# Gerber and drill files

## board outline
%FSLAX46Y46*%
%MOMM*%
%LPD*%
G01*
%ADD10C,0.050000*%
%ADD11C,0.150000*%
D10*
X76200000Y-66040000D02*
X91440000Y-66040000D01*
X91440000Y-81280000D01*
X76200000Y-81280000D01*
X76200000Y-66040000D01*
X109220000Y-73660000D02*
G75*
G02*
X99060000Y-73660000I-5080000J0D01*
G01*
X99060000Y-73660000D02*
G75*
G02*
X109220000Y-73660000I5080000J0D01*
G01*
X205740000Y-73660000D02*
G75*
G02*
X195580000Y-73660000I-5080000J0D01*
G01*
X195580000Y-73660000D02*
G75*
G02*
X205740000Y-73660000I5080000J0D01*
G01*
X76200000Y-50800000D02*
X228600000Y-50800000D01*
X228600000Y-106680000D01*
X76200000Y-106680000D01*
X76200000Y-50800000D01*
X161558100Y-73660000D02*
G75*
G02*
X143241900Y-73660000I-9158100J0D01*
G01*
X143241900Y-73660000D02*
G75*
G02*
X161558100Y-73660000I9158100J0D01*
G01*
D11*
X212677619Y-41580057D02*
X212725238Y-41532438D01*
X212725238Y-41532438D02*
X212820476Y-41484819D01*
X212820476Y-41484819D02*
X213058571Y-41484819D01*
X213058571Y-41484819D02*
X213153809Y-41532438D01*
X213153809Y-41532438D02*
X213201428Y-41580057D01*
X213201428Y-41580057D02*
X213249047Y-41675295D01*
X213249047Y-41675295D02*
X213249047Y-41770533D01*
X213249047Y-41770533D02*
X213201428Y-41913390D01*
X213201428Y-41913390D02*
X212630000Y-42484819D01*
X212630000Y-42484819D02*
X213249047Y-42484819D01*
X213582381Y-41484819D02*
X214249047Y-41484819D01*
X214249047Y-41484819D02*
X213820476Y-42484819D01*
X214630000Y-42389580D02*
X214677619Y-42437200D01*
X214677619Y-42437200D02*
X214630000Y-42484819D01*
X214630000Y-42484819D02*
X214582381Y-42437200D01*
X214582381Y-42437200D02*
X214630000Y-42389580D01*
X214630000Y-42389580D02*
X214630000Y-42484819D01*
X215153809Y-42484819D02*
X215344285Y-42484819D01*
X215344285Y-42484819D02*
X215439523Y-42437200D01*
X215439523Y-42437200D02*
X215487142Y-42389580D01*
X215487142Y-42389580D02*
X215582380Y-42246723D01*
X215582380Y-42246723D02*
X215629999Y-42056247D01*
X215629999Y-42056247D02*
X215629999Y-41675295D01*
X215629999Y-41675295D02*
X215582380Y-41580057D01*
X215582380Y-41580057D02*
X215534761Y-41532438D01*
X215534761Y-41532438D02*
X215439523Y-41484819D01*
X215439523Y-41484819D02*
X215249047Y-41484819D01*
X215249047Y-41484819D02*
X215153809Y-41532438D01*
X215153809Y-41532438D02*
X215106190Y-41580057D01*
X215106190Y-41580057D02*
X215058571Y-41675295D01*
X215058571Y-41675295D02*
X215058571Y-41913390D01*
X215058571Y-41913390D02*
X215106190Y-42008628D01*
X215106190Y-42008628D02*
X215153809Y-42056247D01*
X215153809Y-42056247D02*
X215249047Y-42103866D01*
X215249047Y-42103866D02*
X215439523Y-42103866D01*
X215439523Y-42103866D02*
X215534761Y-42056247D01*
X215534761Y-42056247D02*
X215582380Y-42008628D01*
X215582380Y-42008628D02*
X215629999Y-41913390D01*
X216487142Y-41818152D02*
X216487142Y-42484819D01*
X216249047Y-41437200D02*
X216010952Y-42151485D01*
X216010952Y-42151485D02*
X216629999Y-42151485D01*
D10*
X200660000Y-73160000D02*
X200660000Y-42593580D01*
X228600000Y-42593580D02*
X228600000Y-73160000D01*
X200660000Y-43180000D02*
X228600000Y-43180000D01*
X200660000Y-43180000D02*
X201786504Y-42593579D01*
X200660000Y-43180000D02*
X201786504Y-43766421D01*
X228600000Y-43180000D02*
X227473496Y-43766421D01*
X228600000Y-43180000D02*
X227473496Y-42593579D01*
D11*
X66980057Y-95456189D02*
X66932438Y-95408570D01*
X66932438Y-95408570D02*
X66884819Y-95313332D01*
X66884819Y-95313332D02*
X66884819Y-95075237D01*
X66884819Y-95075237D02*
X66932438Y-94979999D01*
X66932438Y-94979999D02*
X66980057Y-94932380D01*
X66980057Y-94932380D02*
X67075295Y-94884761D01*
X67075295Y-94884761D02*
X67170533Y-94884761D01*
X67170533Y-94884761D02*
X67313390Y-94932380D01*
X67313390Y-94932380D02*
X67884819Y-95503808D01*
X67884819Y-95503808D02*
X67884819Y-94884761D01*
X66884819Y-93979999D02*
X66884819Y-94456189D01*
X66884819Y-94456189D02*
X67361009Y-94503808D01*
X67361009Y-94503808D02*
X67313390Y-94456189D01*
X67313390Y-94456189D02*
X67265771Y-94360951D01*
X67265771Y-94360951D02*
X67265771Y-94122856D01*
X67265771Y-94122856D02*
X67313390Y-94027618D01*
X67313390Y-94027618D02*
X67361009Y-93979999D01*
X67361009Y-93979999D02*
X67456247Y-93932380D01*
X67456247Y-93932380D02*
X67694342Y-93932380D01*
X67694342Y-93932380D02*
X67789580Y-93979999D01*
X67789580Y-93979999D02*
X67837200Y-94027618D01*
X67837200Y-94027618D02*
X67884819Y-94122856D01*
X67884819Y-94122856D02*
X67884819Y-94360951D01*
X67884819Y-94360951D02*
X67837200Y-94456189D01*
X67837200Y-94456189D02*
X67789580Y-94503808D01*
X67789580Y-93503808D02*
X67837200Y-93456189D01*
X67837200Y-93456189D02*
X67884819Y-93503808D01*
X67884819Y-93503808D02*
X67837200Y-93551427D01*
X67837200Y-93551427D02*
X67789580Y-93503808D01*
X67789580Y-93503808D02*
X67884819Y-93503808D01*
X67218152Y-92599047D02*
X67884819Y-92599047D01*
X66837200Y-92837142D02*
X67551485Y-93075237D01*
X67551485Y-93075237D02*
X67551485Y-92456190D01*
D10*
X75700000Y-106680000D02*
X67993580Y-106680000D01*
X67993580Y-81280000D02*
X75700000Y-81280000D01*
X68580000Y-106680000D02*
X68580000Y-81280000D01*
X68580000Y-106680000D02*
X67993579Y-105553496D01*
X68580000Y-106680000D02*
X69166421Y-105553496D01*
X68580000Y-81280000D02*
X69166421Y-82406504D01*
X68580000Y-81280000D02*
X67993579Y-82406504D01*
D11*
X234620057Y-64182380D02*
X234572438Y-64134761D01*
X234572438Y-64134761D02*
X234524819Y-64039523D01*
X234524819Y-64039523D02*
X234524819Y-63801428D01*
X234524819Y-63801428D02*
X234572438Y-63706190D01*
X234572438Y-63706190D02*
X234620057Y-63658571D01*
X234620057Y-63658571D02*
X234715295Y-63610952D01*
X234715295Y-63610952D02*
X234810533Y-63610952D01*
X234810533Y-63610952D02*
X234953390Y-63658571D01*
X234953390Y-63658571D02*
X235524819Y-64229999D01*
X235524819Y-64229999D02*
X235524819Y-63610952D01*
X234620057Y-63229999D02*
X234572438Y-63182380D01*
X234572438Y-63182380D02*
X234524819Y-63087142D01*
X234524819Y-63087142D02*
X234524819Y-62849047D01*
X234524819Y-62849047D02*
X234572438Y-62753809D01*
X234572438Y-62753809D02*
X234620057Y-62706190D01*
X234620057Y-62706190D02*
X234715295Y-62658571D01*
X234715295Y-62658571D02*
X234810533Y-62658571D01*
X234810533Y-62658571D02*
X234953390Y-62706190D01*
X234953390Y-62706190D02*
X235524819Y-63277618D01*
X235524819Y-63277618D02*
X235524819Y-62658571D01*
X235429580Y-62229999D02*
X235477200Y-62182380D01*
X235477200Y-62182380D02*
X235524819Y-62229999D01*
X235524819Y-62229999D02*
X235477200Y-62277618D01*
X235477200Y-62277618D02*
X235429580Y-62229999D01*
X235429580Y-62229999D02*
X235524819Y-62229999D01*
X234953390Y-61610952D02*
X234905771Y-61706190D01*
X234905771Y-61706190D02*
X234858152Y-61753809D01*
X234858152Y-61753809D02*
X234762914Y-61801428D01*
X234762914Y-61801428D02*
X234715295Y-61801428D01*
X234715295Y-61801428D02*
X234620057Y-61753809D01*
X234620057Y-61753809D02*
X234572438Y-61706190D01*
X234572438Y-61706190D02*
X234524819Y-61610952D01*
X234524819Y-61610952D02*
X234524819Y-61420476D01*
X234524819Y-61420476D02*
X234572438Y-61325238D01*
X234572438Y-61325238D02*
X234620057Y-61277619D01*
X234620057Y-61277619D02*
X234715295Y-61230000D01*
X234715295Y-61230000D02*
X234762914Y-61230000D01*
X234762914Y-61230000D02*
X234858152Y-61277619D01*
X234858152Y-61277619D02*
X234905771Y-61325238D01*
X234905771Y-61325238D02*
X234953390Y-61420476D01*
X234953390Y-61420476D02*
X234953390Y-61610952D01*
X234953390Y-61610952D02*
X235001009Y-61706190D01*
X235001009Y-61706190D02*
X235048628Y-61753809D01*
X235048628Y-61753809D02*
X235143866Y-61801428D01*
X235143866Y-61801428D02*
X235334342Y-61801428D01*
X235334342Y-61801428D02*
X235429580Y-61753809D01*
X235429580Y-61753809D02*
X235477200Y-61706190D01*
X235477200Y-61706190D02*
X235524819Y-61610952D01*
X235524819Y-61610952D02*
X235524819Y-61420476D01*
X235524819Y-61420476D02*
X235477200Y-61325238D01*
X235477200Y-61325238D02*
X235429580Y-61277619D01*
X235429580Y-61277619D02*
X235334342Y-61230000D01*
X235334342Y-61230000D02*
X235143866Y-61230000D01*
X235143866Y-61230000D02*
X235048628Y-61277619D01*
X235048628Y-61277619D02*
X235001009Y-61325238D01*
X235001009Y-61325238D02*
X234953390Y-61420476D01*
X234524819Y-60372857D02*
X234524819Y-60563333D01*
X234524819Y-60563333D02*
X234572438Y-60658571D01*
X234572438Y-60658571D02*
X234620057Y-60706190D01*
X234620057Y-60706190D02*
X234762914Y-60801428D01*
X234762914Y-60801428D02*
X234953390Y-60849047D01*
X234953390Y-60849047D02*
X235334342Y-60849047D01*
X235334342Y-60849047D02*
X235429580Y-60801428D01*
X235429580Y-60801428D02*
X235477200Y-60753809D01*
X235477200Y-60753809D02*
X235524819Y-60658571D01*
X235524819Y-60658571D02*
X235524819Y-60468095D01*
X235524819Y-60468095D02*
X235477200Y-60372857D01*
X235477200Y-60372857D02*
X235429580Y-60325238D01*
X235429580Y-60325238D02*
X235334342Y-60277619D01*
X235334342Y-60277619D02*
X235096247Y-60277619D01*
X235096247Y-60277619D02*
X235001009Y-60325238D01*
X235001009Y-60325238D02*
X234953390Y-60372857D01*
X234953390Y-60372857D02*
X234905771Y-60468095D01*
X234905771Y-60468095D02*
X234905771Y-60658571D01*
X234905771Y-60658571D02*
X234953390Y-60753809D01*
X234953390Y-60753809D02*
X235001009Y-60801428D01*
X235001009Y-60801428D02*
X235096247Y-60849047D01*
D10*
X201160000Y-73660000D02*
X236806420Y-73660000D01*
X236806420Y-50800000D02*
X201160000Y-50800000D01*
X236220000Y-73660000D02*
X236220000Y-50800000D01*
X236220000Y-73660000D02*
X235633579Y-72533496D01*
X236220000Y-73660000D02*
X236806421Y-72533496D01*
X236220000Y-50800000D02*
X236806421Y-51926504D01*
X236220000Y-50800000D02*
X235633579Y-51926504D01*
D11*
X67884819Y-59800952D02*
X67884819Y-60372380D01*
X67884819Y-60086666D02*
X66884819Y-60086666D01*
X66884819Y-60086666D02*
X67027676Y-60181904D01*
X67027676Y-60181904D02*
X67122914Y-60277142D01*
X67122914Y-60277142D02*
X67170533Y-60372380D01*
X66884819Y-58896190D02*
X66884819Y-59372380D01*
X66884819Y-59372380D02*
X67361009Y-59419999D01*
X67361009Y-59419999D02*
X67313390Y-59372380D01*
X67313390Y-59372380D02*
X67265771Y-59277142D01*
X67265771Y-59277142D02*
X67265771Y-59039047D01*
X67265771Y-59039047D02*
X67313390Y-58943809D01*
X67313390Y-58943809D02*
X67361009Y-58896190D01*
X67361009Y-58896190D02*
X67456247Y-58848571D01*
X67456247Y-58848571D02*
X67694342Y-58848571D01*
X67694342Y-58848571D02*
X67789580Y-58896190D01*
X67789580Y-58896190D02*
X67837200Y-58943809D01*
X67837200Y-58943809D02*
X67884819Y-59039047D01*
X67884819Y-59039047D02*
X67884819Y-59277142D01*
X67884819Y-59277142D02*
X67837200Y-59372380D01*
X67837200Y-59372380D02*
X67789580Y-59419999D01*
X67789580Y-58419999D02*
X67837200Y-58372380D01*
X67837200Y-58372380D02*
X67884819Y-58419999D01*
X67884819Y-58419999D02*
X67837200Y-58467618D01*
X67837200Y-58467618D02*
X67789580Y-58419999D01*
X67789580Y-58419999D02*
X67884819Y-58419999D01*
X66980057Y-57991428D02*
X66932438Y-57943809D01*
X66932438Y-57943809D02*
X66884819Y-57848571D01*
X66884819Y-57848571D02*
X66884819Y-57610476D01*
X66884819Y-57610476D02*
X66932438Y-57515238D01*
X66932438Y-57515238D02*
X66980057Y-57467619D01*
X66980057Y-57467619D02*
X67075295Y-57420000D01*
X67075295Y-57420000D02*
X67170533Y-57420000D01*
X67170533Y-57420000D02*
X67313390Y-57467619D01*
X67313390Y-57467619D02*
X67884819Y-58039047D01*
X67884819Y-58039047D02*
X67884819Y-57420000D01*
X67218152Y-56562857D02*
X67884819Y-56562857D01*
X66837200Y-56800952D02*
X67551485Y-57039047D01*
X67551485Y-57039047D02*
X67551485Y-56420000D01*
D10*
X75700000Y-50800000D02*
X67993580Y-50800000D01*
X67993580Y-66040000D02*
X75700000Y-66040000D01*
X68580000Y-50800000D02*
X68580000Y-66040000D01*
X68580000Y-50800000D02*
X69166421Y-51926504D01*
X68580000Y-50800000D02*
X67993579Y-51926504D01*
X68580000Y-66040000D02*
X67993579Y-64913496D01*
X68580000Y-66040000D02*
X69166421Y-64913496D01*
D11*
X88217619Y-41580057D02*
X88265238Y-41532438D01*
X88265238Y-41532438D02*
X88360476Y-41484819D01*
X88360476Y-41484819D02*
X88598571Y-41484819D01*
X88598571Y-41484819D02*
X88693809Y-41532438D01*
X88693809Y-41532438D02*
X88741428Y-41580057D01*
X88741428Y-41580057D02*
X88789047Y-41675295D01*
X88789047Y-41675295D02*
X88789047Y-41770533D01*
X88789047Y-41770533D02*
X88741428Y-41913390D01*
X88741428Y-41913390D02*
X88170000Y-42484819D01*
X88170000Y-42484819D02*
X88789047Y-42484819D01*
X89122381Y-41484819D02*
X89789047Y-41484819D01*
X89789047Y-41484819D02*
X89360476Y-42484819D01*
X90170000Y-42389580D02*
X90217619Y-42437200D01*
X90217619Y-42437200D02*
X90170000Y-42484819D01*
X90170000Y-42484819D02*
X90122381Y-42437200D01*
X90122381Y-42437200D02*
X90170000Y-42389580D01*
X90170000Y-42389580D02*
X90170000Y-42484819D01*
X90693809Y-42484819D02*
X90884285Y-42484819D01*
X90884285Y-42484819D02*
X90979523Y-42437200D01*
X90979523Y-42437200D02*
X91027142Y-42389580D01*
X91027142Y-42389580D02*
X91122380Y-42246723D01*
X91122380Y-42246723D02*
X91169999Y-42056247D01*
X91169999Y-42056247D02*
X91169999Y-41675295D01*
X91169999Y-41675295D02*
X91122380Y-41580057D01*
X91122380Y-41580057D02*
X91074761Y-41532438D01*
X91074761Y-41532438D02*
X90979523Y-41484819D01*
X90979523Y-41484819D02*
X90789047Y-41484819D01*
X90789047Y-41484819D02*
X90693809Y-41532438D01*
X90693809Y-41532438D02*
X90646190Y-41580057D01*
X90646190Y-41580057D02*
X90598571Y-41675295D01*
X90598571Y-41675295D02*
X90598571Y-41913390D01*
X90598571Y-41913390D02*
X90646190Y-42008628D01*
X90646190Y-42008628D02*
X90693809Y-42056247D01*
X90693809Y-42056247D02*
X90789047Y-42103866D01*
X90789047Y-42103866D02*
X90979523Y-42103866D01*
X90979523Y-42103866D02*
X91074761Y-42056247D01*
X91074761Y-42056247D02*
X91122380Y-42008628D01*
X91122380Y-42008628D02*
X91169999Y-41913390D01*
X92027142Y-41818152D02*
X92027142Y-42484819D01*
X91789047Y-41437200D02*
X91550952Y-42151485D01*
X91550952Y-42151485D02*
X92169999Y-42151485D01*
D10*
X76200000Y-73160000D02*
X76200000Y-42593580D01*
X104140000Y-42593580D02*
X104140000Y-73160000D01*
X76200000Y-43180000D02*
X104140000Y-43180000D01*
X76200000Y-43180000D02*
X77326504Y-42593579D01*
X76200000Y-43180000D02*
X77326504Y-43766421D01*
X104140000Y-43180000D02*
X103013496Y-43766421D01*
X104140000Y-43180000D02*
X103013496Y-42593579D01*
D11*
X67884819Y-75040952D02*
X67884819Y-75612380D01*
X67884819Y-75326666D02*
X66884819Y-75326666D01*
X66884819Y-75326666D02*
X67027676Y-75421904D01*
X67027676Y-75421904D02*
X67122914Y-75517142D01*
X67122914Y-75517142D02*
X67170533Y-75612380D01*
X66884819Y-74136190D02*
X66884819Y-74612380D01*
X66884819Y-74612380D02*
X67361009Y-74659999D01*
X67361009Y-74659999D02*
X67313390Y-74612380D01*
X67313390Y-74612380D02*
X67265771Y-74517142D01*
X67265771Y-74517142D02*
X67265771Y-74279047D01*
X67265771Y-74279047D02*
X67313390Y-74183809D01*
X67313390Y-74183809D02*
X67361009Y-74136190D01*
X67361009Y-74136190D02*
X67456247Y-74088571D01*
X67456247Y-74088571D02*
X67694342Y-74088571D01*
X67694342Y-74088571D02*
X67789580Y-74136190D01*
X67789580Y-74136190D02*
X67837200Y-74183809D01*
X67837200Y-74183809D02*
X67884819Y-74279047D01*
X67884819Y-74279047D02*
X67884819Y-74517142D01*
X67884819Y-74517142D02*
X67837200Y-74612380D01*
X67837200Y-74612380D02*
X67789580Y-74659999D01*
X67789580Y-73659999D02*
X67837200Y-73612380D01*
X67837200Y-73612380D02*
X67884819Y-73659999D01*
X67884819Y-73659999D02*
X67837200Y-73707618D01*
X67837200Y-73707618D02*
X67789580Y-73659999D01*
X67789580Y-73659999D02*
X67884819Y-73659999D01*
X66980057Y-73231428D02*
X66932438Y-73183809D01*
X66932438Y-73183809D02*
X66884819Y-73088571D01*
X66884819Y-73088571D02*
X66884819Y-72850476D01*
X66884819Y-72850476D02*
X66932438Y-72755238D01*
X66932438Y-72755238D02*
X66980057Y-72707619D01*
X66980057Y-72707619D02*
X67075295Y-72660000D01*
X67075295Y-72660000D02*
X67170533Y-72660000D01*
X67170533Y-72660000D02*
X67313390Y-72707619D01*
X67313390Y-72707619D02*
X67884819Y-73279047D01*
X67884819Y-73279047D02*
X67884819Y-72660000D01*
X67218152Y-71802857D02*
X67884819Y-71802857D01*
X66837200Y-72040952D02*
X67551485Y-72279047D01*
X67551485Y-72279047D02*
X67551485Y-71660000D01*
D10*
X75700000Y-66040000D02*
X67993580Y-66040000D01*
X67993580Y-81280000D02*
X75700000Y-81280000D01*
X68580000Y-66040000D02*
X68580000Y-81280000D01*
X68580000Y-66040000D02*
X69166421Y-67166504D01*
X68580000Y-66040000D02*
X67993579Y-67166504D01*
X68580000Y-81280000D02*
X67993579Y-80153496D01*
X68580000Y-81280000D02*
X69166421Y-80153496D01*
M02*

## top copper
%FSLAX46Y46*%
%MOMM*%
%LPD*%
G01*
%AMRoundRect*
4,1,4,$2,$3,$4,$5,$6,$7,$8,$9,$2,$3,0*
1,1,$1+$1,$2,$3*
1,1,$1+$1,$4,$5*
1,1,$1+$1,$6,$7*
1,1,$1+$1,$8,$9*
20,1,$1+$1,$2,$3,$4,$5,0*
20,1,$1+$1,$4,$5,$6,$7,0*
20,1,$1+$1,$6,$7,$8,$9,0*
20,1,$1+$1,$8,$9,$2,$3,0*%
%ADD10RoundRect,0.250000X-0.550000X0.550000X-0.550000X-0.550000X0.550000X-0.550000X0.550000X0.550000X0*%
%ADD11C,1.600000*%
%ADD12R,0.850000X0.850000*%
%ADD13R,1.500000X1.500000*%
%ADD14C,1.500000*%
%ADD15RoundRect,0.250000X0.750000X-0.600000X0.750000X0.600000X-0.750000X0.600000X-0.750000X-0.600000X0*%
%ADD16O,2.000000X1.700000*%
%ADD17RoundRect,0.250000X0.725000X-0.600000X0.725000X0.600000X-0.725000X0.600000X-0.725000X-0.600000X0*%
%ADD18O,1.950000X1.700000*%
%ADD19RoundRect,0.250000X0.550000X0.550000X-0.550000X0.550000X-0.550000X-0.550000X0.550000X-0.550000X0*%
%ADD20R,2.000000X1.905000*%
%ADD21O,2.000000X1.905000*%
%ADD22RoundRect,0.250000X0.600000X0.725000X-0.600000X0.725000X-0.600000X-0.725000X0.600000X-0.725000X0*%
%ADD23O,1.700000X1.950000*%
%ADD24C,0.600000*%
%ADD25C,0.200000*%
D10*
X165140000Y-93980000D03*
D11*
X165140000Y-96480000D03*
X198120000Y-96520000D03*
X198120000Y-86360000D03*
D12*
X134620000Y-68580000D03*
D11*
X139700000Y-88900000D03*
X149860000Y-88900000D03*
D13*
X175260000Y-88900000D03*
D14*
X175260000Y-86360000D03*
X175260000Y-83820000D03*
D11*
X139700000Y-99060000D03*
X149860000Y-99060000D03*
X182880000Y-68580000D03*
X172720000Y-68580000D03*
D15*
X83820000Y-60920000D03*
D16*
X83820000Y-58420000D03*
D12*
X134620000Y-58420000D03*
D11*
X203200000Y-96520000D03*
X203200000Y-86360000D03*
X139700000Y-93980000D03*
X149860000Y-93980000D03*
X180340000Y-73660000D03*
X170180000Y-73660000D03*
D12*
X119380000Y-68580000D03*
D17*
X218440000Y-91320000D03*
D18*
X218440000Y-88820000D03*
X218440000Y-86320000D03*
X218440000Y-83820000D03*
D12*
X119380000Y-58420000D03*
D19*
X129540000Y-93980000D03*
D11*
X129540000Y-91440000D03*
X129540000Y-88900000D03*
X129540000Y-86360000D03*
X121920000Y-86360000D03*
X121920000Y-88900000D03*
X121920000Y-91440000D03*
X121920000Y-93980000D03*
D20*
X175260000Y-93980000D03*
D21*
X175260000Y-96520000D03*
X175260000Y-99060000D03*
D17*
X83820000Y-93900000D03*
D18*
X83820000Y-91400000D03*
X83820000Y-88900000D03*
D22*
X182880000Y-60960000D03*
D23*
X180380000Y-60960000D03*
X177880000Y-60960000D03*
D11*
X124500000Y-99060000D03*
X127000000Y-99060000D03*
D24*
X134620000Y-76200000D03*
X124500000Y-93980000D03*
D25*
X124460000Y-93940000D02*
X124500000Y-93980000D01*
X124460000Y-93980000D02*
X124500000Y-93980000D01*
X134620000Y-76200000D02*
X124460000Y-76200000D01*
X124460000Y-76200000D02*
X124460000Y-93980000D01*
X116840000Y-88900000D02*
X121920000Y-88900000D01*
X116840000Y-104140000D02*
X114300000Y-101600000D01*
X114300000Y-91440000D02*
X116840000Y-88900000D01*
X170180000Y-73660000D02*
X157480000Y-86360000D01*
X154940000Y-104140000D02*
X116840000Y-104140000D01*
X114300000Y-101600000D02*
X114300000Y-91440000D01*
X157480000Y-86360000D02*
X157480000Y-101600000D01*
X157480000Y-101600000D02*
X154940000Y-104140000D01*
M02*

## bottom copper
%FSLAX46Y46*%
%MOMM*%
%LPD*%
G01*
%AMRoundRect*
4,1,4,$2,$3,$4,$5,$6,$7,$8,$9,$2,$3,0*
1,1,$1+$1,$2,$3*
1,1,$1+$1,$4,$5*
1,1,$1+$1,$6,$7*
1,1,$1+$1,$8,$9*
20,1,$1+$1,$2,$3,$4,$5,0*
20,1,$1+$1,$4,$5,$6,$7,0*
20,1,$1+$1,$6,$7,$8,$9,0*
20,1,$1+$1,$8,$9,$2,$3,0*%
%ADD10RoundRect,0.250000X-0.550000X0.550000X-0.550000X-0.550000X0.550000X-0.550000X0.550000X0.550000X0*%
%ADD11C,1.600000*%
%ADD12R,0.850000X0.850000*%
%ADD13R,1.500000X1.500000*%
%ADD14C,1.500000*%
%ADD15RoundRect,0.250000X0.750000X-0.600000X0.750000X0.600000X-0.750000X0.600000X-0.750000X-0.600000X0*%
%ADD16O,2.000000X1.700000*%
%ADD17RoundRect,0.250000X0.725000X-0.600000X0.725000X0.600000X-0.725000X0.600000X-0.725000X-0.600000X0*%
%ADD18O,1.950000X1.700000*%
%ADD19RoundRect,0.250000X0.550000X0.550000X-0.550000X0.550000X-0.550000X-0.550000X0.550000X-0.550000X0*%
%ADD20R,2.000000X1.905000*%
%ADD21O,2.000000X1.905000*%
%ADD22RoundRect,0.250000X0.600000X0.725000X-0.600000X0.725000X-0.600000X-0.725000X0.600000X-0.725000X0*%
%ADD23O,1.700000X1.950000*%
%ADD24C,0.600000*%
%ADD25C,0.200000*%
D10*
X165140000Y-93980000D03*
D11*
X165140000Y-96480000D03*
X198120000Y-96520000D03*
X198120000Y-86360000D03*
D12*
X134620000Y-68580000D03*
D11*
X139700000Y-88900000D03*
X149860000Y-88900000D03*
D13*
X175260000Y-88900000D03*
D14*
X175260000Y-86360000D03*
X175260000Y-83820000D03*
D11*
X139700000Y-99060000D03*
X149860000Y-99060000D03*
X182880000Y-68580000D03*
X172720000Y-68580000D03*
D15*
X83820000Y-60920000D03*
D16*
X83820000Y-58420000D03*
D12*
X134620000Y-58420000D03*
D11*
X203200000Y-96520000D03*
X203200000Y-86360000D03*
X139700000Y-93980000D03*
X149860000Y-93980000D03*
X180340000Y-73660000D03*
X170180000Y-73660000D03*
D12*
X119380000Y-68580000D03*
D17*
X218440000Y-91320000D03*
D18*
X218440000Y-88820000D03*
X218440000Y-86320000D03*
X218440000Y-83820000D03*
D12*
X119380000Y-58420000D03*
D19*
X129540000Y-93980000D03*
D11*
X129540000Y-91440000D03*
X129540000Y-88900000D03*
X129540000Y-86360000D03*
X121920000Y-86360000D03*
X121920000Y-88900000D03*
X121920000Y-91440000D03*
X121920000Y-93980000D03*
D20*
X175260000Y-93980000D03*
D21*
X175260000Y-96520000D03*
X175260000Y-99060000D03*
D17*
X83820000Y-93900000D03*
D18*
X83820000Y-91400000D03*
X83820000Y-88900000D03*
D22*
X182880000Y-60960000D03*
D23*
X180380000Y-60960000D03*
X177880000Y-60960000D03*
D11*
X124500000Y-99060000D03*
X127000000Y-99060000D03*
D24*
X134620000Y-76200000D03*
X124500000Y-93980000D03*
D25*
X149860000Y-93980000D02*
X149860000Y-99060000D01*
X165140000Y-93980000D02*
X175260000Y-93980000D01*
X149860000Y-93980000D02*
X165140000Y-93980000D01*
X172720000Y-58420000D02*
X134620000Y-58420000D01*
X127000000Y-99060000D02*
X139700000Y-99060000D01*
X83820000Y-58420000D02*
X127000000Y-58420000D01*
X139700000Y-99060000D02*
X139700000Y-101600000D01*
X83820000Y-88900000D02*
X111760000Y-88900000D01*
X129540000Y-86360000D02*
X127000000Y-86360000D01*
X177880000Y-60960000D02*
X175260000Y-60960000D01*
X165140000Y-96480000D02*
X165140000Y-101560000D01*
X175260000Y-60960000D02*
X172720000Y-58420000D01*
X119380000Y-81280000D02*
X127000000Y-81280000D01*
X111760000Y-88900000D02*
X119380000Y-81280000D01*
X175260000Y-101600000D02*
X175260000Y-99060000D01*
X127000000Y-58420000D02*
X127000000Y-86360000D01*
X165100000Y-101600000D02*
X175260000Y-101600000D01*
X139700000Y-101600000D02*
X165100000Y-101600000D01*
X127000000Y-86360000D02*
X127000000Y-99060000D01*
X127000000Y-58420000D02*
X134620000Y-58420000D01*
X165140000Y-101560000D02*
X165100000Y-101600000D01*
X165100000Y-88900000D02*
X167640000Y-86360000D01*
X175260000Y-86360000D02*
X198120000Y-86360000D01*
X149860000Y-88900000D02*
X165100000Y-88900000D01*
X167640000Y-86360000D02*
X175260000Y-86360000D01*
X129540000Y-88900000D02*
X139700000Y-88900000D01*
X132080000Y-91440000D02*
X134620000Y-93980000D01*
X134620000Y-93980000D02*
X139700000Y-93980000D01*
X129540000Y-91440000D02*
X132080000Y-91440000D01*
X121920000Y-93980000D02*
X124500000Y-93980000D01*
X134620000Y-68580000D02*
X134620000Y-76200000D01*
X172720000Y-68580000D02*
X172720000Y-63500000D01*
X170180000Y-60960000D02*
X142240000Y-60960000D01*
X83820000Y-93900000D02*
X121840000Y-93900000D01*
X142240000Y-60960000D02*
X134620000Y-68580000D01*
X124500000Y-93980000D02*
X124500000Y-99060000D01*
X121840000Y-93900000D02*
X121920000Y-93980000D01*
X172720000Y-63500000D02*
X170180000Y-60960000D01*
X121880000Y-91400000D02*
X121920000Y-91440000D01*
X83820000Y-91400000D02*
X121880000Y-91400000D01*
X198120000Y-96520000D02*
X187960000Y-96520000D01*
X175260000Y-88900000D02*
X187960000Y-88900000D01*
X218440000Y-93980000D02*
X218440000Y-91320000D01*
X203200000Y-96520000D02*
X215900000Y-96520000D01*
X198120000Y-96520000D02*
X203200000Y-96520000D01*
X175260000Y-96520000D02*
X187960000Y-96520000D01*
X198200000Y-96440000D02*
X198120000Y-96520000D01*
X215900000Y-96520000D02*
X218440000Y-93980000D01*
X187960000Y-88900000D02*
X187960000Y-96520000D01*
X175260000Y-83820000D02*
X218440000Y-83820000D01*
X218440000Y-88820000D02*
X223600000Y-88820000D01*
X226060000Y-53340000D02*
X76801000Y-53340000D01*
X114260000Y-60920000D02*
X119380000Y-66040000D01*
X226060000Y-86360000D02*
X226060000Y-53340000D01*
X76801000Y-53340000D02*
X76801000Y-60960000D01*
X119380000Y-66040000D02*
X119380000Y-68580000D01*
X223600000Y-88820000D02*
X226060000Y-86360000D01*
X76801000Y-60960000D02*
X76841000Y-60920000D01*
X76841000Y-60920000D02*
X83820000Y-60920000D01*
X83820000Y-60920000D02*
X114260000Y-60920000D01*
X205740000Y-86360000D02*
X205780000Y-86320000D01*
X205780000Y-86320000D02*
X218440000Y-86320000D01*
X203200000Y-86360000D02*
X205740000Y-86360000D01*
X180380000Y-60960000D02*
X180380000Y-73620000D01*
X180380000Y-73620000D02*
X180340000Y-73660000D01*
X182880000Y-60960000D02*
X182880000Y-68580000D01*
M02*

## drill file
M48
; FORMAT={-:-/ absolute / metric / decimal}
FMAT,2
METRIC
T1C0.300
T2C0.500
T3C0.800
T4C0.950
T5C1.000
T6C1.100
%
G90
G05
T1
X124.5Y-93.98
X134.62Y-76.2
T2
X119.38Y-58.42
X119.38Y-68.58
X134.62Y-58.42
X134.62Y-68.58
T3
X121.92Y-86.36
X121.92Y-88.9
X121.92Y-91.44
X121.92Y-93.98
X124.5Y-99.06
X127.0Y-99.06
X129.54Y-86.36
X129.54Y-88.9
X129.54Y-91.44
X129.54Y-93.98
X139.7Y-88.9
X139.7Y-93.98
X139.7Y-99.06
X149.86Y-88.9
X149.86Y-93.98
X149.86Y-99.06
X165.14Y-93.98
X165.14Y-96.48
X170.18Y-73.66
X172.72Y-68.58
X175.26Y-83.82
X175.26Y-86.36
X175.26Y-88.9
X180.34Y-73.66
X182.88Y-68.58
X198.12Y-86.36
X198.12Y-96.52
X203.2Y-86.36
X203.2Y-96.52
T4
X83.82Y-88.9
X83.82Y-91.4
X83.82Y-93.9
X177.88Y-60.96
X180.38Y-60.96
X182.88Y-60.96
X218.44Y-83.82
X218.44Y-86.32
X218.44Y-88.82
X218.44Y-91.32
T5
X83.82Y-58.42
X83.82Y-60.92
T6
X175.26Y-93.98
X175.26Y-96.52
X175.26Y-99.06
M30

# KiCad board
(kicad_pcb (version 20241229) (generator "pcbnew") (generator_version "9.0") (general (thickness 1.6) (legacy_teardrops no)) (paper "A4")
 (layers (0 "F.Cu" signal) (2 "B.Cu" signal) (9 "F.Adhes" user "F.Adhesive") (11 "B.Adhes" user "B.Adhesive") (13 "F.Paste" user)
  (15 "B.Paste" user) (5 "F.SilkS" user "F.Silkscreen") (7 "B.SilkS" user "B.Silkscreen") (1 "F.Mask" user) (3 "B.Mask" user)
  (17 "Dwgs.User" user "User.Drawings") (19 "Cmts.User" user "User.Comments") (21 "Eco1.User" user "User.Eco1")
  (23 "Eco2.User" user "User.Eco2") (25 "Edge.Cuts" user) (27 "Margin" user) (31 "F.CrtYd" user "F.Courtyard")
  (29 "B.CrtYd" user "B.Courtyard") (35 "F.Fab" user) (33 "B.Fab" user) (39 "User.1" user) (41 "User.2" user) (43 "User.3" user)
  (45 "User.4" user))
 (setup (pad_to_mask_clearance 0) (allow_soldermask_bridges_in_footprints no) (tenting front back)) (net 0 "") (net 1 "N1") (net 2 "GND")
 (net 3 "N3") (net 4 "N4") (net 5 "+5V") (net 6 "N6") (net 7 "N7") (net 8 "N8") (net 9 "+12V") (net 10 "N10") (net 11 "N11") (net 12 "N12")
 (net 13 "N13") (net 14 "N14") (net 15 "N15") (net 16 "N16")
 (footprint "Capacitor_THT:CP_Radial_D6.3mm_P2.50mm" (layer "F.Cu") (at 165.14 93.98 -90)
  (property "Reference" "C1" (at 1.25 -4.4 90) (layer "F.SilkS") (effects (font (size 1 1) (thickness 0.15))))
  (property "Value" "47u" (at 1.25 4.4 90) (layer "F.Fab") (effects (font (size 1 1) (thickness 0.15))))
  (pad "1" thru_hole roundrect (at 0 0 270) (size 1.6 1.6) (drill 0.8) (layers "*.Cu" "*.Mask") (remove_unused_layers no)
   (roundrect_rratio 0.15625) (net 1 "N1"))
  (pad "2" thru_hole circle (at 2.5 0 270) (size 1.6 1.6) (drill 0.8) (layers "*.Cu" "*.Mask") (remove_unused_layers no) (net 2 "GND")))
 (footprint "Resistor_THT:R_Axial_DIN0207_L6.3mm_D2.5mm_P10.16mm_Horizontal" (layer "F.Cu") (at 198.12 96.52 90)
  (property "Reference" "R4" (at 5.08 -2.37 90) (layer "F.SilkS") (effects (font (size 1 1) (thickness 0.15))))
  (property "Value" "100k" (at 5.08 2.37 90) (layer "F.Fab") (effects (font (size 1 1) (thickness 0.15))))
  (pad "1" thru_hole circle (at 0 0 90) (size 1.6 1.6) (drill 0.8) (layers "*.Cu" "*.Mask") (remove_unused_layers no) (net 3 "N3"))
  (pad "2" thru_hole circle (at 10.16 0 90) (size 1.6 1.6) (drill 0.8) (layers "*.Cu" "*.Mask") (remove_unused_layers no) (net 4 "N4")))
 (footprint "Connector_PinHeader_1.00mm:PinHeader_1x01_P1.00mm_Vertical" (layer "F.Cu") (at 134.62 68.58)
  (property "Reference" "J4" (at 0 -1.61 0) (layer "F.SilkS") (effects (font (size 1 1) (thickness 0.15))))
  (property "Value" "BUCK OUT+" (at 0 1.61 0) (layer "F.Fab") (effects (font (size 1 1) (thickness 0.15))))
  (pad "1" thru_hole rect (at 0 0) (size 0.85 0.85) (drill 0.5) (layers "*.Cu" "*.Mask") (remove_unused_layers no) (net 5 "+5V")))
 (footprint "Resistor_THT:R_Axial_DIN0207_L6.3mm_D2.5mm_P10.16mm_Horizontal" (layer "F.Cu") (at 139.7 88.9)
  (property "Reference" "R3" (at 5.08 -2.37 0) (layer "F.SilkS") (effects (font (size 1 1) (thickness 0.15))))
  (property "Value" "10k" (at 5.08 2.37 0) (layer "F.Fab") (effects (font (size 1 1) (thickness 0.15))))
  (pad "1" thru_hole circle (at 0 0) (size 1.6 1.6) (drill 0.8) (layers "*.Cu" "*.Mask") (remove_unused_layers no) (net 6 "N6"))
  (pad "2" thru_hole circle (at 10.16 0) (size 1.6 1.6) (drill 0.8) (layers "*.Cu" "*.Mask") (remove_unused_layers no) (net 4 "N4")))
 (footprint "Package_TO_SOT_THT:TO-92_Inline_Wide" (layer "F.Cu") (at 175.26 88.9 90)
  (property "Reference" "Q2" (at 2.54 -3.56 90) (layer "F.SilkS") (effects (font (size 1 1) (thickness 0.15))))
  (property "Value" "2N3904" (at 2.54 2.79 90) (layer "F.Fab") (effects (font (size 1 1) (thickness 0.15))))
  (pad "1" thru_hole rect (at 0 0 90) (size 1.5 1.5) (drill 0.8) (layers "*.Cu" "*.Mask") (remove_unused_layers no) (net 3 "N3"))
  (pad "2" thru_hole circle (at 2.54 0 90) (size 1.5 1.5) (drill 0.8) (layers "*.Cu" "*.Mask") (remove_unused_layers no) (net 4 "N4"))
  (pad "3" thru_hole circle (at 5.08 0 90) (size 1.5 1.5) (drill 0.8) (layers "*.Cu" "*.Mask") (remove_unused_layers no) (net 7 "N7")))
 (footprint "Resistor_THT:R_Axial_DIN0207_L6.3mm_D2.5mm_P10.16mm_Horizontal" (layer "F.Cu") (at 139.7 99.06)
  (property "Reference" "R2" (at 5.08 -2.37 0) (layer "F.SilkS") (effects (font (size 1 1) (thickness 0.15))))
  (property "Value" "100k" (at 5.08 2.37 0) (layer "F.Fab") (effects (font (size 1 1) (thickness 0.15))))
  (pad "1" thru_hole circle (at 0 0) (size 1.6 1.6) (drill 0.8) (layers "*.Cu" "*.Mask") (remove_unused_layers no) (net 2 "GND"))
  (pad "2" thru_hole circle (at 10.16 0) (size 1.6 1.6) (drill 0.8) (layers "*.Cu" "*.Mask") (remove_unused_layers no) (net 1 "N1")))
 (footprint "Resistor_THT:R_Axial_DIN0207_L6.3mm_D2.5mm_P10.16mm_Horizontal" (layer "F.Cu") (at 182.88 68.58 180)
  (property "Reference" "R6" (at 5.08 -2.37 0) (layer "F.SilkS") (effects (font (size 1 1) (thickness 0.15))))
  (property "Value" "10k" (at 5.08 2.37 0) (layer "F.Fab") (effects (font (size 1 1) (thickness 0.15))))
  (pad "1" thru_hole circle (at 0 0 180) (size 1.6 1.6) (drill 0.8) (layers "*.Cu" "*.Mask") (remove_unused_layers no) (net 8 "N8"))
  (pad "2" thru_hole circle (at 10.16 0 180) (size 1.6 1.6) (drill 0.8) (layers "*.Cu" "*.Mask") (remove_unused_layers no) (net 5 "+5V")))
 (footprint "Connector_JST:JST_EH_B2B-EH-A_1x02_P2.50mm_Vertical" (layer "F.Cu") (at 83.82 60.92 90)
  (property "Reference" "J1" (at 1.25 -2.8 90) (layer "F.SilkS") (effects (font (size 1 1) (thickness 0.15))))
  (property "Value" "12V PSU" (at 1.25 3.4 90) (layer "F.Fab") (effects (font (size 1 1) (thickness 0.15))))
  (pad "1" thru_hole roundrect (at 0 0 90) (size 1.7 2) (drill 1) (layers "*.Cu" "*.Mask") (remove_unused_layers no)
   (roundrect_rratio 0.147059) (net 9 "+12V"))
  (pad "2" thru_hole oval (at 2.5 0 90) (size 1.7 2) (drill 1) (layers "*.Cu" "*.Mask") (remove_unused_layers no) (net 2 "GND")))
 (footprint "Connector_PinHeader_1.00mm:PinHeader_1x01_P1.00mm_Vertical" (layer "F.Cu") (at 134.62 58.42)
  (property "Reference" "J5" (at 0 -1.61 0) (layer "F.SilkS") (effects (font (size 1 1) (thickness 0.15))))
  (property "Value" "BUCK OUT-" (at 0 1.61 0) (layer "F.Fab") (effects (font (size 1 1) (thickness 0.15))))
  (pad "1" thru_hole rect (at 0 0) (size 0.85 0.85) (drill 0.5) (layers "*.Cu" "*.Mask") (remove_unused_layers no) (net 2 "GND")))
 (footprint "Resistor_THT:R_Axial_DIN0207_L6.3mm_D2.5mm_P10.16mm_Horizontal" (layer "F.Cu") (at 203.2 96.52 90)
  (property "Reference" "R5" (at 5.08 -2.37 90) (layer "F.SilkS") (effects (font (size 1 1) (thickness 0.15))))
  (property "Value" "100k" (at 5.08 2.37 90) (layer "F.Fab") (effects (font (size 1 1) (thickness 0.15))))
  (pad "1" thru_hole circle (at 0 0 90) (size 1.6 1.6) (drill 0.8) (layers "*.Cu" "*.Mask") (remove_unused_layers no) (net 3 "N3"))
  (pad "2" thru_hole circle (at 10.16 0 90) (size 1.6 1.6) (drill 0.8) (layers "*.Cu" "*.Mask") (remove_unused_layers no) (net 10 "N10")))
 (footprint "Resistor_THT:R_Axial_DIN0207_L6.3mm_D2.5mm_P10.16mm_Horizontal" (layer "F.Cu") (at 139.7 93.98)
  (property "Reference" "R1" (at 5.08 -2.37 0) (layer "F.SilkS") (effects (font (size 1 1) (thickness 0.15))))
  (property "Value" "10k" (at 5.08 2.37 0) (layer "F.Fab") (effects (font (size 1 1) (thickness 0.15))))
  (pad "1" thru_hole circle (at 0 0) (size 1.6 1.6) (drill 0.8) (layers "*.Cu" "*.Mask") (remove_unused_layers no) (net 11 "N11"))
  (pad "2" thru_hole circle (at 10.16 0) (size 1.6 1.6) (drill 0.8) (layers "*.Cu" "*.Mask") (remove_unused_layers no) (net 1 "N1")))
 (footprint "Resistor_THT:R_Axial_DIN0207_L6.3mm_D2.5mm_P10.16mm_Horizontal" (layer "F.Cu") (at 180.34 73.66 180)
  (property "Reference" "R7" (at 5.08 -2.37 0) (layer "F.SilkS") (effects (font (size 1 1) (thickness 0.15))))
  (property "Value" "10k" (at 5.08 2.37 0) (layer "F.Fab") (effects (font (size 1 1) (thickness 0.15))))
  (pad "1" thru_hole circle (at 0 0 180) (size 1.6 1.6) (drill 0.8) (layers "*.Cu" "*.Mask") (remove_unused_layers no) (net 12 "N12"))
  (pad "2" thru_hole circle (at 10.16 0 180) (size 1.6 1.6) (drill 0.8) (layers "*.Cu" "*.Mask") (remove_unused_layers no) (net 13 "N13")))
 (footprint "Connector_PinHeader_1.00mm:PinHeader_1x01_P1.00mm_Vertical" (layer "F.Cu") (at 119.38 68.58)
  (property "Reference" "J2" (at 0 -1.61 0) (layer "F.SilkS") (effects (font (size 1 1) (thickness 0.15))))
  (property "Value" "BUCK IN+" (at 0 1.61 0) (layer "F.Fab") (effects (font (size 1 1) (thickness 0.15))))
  (pad "1" thru_hole rect (at 0 0) (size 0.85 0.85) (drill 0.5) (layers "*.Cu" "*.Mask") (remove_unused_layers no) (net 9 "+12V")))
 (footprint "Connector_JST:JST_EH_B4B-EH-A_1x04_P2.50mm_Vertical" (layer "F.Cu") (at 218.44 91.32 90)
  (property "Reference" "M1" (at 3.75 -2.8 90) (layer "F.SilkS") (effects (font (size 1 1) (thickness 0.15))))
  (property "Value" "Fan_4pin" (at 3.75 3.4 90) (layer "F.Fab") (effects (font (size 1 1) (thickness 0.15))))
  (pad "1" thru_hole roundrect (at 0 0 90) (size 1.7 1.95) (drill 0.95) (layers "*.Cu" "*.Mask") (remove_unused_layers no)
   (roundrect_rratio 0.147059) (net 3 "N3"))
  (pad "2" thru_hole oval (at 2.5 0 90) (size 1.7 1.95) (drill 0.95) (layers "*.Cu" "*.Mask") (remove_unused_layers no) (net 9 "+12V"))
  (pad "3" thru_hole oval (at 5 0 90) (size 1.7 1.95) (drill 0.95) (layers "*.Cu" "*.Mask") (remove_unused_layers no) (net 10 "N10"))
  (pad "4" thru_hole oval (at 7.5 0 90) (size 1.7 1.95) (drill 0.95) (layers "*.Cu" "*.Mask") (remove_unused_layers no) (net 7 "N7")))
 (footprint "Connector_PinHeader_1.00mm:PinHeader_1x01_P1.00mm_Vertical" (layer "F.Cu") (at 119.38 58.42)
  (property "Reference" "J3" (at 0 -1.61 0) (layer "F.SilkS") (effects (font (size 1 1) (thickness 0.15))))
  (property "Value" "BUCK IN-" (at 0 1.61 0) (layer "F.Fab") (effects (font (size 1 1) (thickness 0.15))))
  (pad "1" thru_hole rect (at 0 0) (size 0.85 0.85) (drill 0.5) (layers "*.Cu" "*.Mask") (remove_unused_layers no) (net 2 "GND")))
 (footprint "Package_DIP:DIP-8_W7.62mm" (layer "F.Cu") (at 129.54 93.98 180)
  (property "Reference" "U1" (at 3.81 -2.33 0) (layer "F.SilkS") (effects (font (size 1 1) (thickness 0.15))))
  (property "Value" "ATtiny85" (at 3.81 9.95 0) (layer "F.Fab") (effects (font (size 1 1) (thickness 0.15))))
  (pad "1" thru_hole roundrect (at 0 0 180) (size 1.6 1.6) (drill 0.8) (layers "*.Cu" "*.Mask") (remove_unused_layers no)
   (roundrect_rratio 0.15625) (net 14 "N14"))
  (pad "2" thru_hole circle (at 0 2.54 180) (size 1.6 1.6) (drill 0.8) (layers "*.Cu" "*.Mask") (remove_unused_layers no) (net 11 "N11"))
  (pad "3" thru_hole circle (at 0 5.08 180) (size 1.6 1.6) (drill 0.8) (layers "*.Cu" "*.Mask") (remove_unused_layers no) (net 6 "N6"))
  (pad "4" thru_hole circle (at 0 7.62 180) (size 1.6 1.6) (drill 0.8) (layers "*.Cu" "*.Mask") (remove_unused_layers no) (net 2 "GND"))
  (pad "5" thru_hole circle (at 7.62 7.62 180) (size 1.6 1.6) (drill 0.8) (layers "*.Cu" "*.Mask") (remove_unused_layers no) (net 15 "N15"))
  (pad "6" thru_hole circle (at 7.62 5.08 180) (size 1.6 1.6) (drill 0.8) (layers "*.Cu" "*.Mask") (remove_unused_layers no) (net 13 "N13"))
  (pad "7" thru_hole circle (at 7.62 2.54 180) (size 1.6 1.6) (drill 0.8) (layers "*.Cu" "*.Mask") (remove_unused_layers no) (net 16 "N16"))
  (pad "8" thru_hole circle (at 7.62 0 180) (size 1.6 1.6) (drill 0.8) (layers "*.Cu" "*.Mask") (remove_unused_layers no) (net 5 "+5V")))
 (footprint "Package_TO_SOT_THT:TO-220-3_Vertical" (layer "F.Cu") (at 175.26 93.98 -90)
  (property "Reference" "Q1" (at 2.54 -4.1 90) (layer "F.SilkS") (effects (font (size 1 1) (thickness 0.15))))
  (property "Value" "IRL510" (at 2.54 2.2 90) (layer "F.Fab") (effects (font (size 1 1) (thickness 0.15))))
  (pad "1" thru_hole rect (at 0 0 270) (size 1.905 2) (drill 1.1) (layers "*.Cu" "*.Mask") (remove_unused_layers no) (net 1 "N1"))
  (pad "2" thru_hole oval (at 2.54 0 270) (size 1.905 2) (drill 1.1) (layers "*.Cu" "*.Mask") (remove_unused_layers no) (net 3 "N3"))
  (pad "3" thru_hole oval (at 5.08 0 270) (size 1.905 2) (drill 1.1) (layers "*.Cu" "*.Mask") (remove_unused_layers no) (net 2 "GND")))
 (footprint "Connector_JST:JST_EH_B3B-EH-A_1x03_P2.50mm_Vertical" (layer "F.Cu") (at 83.82 93.9 90)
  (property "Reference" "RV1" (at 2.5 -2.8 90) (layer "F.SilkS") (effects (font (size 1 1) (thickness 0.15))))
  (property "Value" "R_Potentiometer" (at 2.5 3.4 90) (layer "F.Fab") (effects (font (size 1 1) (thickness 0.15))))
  (pad "1" thru_hole roundrect (at 0 0 90) (size 1.7 1.95) (drill 0.95) (layers "*.Cu" "*.Mask") (remove_unused_layers no)
   (roundrect_rratio 0.147059) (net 5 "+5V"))
  (pad "2" thru_hole oval (at 2.5 0 90) (size 1.7 1.95) (drill 0.95) (layers "*.Cu" "*.Mask") (remove_unused_layers no) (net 16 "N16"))
  (pad "3" thru_hole oval (at 5 0 90) (size 1.7 1.95) (drill 0.95) (layers "*.Cu" "*.Mask") (remove_unused_layers no) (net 2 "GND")))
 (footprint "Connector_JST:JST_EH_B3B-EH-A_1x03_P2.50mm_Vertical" (layer "F.Cu") (at 182.88 60.96 180)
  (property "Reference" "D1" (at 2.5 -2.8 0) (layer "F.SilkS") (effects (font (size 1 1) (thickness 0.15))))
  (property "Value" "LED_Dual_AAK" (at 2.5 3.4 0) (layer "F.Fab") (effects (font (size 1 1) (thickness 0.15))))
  (pad "1" thru_hole roundrect (at 0 0 180) (size 1.7 1.95) (drill 0.95) (layers "*.Cu" "*.Mask") (remove_unused_layers no)
   (roundrect_rratio 0.147059) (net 8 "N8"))
  (pad "2" thru_hole oval (at 2.5 0 180) (size 1.7 1.95) (drill 0.95) (layers "*.Cu" "*.Mask") (remove_unused_layers no) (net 12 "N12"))
  (pad "3" thru_hole oval (at 5 0 180) (size 1.7 1.95) (drill 0.95) (layers "*.Cu" "*.Mask") (remove_unused_layers no) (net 2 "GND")))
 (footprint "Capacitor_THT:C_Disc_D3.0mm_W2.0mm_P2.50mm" (layer "F.Cu") (at 124.5 99.06)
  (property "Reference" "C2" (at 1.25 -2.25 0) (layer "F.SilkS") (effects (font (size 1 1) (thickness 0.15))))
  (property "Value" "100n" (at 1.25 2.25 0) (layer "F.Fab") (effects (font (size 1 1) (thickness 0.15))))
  (pad "1" thru_hole circle (at 0 0) (size 1.6 1.6) (drill 0.8) (layers "*.Cu" "*.Mask") (remove_unused_layers no) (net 5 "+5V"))
  (pad "2" thru_hole circle (at 2.5 0) (size 1.6 1.6) (drill 0.8) (layers "*.Cu" "*.Mask") (remove_unused_layers no) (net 2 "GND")))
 (gr_rect (start 76.2 66.04) (end 91.44 81.28) (stroke (width 0.05) (type default)) (fill no) (layer "Edge.Cuts"))
 (gr_circle (center 104.14 73.66) (end 109.22 73.66) (stroke (width 0.05) (type default)) (fill no) (layer "Edge.Cuts"))
 (gr_circle (center 200.66 73.66) (end 205.74 73.66) (stroke (width 0.05) (type default)) (fill no) (layer "Edge.Cuts"))
 (gr_rect (start 76.2 50.8) (end 228.6 106.68) (stroke (width 0.05) (type default)) (fill no) (layer "Edge.Cuts"))
 (gr_circle (center 152.4 73.66) (end 160.02 78.74) (stroke (width 0.05) (type default)) (fill no) (layer "Edge.Cuts"))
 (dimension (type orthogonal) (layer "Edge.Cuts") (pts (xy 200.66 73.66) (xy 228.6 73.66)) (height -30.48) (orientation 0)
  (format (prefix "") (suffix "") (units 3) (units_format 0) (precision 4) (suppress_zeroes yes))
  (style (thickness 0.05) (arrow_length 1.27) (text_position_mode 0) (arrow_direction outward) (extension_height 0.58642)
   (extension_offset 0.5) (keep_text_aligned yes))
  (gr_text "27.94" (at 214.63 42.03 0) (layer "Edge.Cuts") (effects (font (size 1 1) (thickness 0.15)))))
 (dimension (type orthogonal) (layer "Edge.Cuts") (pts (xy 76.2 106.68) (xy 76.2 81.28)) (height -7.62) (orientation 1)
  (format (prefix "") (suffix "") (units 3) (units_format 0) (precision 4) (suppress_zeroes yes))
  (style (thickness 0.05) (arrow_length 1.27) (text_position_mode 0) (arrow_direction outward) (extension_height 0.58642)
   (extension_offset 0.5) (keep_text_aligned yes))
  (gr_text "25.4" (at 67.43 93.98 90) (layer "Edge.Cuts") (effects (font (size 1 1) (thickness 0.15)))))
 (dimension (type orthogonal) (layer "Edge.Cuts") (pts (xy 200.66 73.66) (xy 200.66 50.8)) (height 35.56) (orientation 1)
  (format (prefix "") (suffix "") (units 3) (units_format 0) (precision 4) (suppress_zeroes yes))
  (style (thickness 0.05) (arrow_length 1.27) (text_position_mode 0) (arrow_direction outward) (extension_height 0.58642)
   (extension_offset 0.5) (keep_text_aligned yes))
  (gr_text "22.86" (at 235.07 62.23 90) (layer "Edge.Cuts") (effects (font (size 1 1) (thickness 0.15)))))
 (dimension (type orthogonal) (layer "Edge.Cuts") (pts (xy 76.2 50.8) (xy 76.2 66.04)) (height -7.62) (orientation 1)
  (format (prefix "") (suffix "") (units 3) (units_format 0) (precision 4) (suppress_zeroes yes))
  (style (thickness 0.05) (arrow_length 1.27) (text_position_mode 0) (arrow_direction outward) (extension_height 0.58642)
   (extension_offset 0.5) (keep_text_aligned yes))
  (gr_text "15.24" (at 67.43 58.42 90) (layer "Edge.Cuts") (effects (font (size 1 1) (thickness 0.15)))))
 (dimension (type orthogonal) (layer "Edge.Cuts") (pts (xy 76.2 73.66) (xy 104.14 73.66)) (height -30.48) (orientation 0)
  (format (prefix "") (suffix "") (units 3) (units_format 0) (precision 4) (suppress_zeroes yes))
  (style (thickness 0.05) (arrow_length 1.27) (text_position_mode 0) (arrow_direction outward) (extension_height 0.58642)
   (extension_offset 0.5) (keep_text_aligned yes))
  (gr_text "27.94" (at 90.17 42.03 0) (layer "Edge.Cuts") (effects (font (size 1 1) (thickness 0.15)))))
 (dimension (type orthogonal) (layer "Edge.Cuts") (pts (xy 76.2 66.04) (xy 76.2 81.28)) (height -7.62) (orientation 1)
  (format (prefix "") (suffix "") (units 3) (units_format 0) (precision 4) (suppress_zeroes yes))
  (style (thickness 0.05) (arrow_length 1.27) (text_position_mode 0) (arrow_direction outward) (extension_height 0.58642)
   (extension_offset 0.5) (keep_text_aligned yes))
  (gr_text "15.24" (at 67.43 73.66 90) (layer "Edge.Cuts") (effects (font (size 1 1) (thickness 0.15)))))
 (segment (start 149.86 93.98) (end 149.86 99.06) (width 0.2) (layer "B.Cu") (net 1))
 (segment (start 165.14 93.98) (end 175.26 93.98) (width 0.2) (layer "B.Cu") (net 1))
 (segment (start 149.86 93.98) (end 165.14 93.98) (width 0.2) (layer "B.Cu") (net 1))
 (segment (start 172.72 58.42) (end 134.62 58.42) (width 0.2) (layer "B.Cu") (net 2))
 (segment (start 127 99.06) (end 139.7 99.06) (width 0.2) (layer "B.Cu") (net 2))
 (segment (start 83.82 58.42) (end 127 58.42) (width 0.2) (layer "B.Cu") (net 2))
 (segment (start 139.7 99.06) (end 139.7 101.6) (width 0.2) (layer "B.Cu") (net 2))
 (segment (start 83.82 88.9) (end 111.76 88.9) (width 0.2) (layer "B.Cu") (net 2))
 (segment (start 129.54 86.36) (end 127 86.36) (width 0.2) (layer "B.Cu") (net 2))
 (segment (start 177.88 60.96) (end 175.26 60.96) (width 0.2) (layer "B.Cu") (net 2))
 (segment (start 165.14 96.48) (end 165.14 101.56) (width 0.2) (layer "B.Cu") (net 2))
 (segment (start 175.26 60.96) (end 172.72 58.42) (width 0.2) (layer "B.Cu") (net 2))
 (segment (start 119.38 81.28) (end 127 81.28) (width 0.2) (layer "B.Cu") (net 2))
 (segment (start 111.76 88.9) (end 119.38 81.28) (width 0.2) (layer "B.Cu") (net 2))
 (segment (start 175.26 101.6) (end 175.26 99.06) (width 0.2) (layer "B.Cu") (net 2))
 (segment (start 127 58.42) (end 127 86.36) (width 0.2) (layer "B.Cu") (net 2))
 (segment (start 165.1 101.6) (end 175.26 101.6) (width 0.2) (layer "B.Cu") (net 2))
 (segment (start 139.7 101.6) (end 165.1 101.6) (width 0.2) (layer "B.Cu") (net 2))
 (segment (start 127 86.36) (end 127 99.06) (width 0.2) (layer "B.Cu") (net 2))
 (segment (start 127 58.42) (end 134.62 58.42) (width 0.2) (layer "B.Cu") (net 2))
 (segment (start 165.14 101.56) (end 165.1 101.6) (width 0.2) (layer "B.Cu") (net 2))
 (segment (start 165.1 88.9) (end 167.64 86.36) (width 0.2) (layer "B.Cu") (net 4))
 (segment (start 175.26 86.36) (end 198.12 86.36) (width 0.2) (layer "B.Cu") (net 4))
 (segment (start 149.86 88.9) (end 165.1 88.9) (width 0.2) (layer "B.Cu") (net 4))
 (segment (start 167.64 86.36) (end 175.26 86.36) (width 0.2) (layer "B.Cu") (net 4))
 (segment (start 129.54 88.9) (end 139.7 88.9) (width 0.2) (layer "B.Cu") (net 6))
 (segment (start 132.08 91.44) (end 134.62 93.98) (width 0.2) (layer "B.Cu") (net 11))
 (segment (start 134.62 93.98) (end 139.7 93.98) (width 0.2) (layer "B.Cu") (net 11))
 (segment (start 129.54 91.44) (end 132.08 91.44) (width 0.2) (layer "B.Cu") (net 11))
 (segment (start 124.46 93.94) (end 124.5 93.98) (width 0.2) (layer "F.Cu") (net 5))
 (segment (start 124.46 93.98) (end 124.5 93.98) (width 0.2) (layer "F.Cu") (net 5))
 (segment (start 134.62 76.2) (end 124.46 76.2) (width 0.2) (layer "F.Cu") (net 5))
 (segment (start 124.46 76.2) (end 124.46 93.98) (width 0.2) (layer "F.Cu") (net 5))
 (via (at 134.62 76.2) (size 0.6) (drill 0.3) (layers "F.Cu" "B.Cu") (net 5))
 (via (at 124.5 93.98) (size 0.6) (drill 0.3) (layers "F.Cu" "B.Cu") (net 5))
 (segment (start 121.92 93.98) (end 124.5 93.98) (width 0.2) (layer "B.Cu") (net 5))
 (segment (start 134.62 68.58) (end 134.62 76.2) (width 0.2) (layer "B.Cu") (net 5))
 (segment (start 172.72 68.58) (end 172.72 63.5) (width 0.2) (layer "B.Cu") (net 5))
 (segment (start 170.18 60.96) (end 142.24 60.96) (width 0.2) (layer "B.Cu") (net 5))
 (segment (start 83.82 93.9) (end 121.84 93.9) (width 0.2) (layer "B.Cu") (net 5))
 (segment (start 142.24 60.96) (end 134.62 68.58) (width 0.2) (layer "B.Cu") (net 5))
 (segment (start 124.5 93.98) (end 124.5 99.06) (width 0.2) (layer "B.Cu") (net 5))
 (segment (start 121.84 93.9) (end 121.92 93.98) (width 0.2) (layer "B.Cu") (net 5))
 (segment (start 172.72 63.5) (end 170.18 60.96) (width 0.2) (layer "B.Cu") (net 5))
 (segment (start 121.88 91.4) (end 121.92 91.44) (width 0.2) (layer "B.Cu") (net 16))
 (segment (start 83.82 91.4) (end 121.88 91.4) (width 0.2) (layer "B.Cu") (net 16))
 (segment (start 198.12 96.52) (end 187.96 96.52) (width 0.2) (layer "B.Cu") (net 3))
 (segment (start 175.26 88.9) (end 187.96 88.9) (width 0.2) (layer "B.Cu") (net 3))
 (segment (start 218.44 93.98) (end 218.44 91.32) (width 0.2) (layer "B.Cu") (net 3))
 (segment (start 203.2 96.52) (end 215.9 96.52) (width 0.2) (layer "B.Cu") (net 3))
 (segment (start 198.12 96.52) (end 203.2 96.52) (width 0.2) (layer "B.Cu") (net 3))
 (segment (start 175.26 96.52) (end 187.96 96.52) (width 0.2) (layer "B.Cu") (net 3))
 (segment (start 198.2 96.44) (end 198.12 96.52) (width 0.2) (layer "B.Cu") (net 3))
 (segment (start 215.9 96.52) (end 218.44 93.98) (width 0.2) (layer "B.Cu") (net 3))
 (segment (start 187.96 88.9) (end 187.96 96.52) (width 0.2) (layer "B.Cu") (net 3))
 (segment (start 175.26 83.82) (end 218.44 83.82) (width 0.2) (layer "B.Cu") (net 7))
 (segment (start 218.44 88.82) (end 223.6 88.82) (width 0.2) (layer "B.Cu") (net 9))
 (segment (start 226.06 53.34) (end 76.801 53.34) (width 0.2) (layer "B.Cu") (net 9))
 (segment (start 114.26 60.92) (end 119.38 66.04) (width 0.2) (layer "B.Cu") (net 9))
 (segment (start 226.06 86.36) (end 226.06 53.34) (width 0.2) (layer "B.Cu") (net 9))
 (segment (start 76.801 53.34) (end 76.801 60.96) (width 0.2) (layer "B.Cu") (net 9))
 (segment (start 119.38 66.04) (end 119.38 68.58) (width 0.2) (layer "B.Cu") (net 9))
 (segment (start 223.6 88.82) (end 226.06 86.36) (width 0.2) (layer "B.Cu") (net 9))
 (segment (start 76.801 60.96) (end 76.841 60.92) (width 0.2) (layer "B.Cu") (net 9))
 (segment (start 76.841 60.92) (end 83.82 60.92) (width 0.2) (layer "B.Cu") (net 9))
 (segment (start 83.82 60.92) (end 114.26 60.92) (width 0.2) (layer "B.Cu") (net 9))
 (segment (start 205.74 86.36) (end 205.78 86.32) (width 0.2) (layer "B.Cu") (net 10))
 (segment (start 205.78 86.32) (end 218.44 86.32) (width 0.2) (layer "B.Cu") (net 10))
 (segment (start 203.2 86.36) (end 205.74 86.36) (width 0.2) (layer "B.Cu") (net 10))
 (segment (start 180.38 60.96) (end 180.38 73.62) (width 0.2) (layer "B.Cu") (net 12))
 (segment (start 180.38 73.62) (end 180.34 73.66) (width 0.2) (layer "B.Cu") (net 12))
 (segment (start 182.88 60.96) (end 182.88 68.58) (width 0.2) (layer "B.Cu") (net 8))
 (segment (start 116.84 88.9) (end 121.92 88.9) (width 0.2) (layer "F.Cu") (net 13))
 (segment (start 116.84 104.14) (end 114.3 101.6) (width 0.2) (layer "F.Cu") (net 13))
 (segment (start 114.3 91.44) (end 116.84 88.9) (width 0.2) (layer "F.Cu") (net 13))
 (segment (start 170.18 73.66) (end 157.48 86.36) (width 0.2) (layer "F.Cu") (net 13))
 (segment (start 154.94 104.14) (end 116.84 104.14) (width 0.2) (layer "F.Cu") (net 13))
 (segment (start 114.3 101.6) (end 114.3 91.44) (width 0.2) (layer "F.Cu") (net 13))
 (segment (start 157.48 86.36) (end 157.48 101.6) (width 0.2) (layer "F.Cu") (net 13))
 (segment (start 157.48 101.6) (end 154.94 104.14) (width 0.2) (layer "F.Cu") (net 13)))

